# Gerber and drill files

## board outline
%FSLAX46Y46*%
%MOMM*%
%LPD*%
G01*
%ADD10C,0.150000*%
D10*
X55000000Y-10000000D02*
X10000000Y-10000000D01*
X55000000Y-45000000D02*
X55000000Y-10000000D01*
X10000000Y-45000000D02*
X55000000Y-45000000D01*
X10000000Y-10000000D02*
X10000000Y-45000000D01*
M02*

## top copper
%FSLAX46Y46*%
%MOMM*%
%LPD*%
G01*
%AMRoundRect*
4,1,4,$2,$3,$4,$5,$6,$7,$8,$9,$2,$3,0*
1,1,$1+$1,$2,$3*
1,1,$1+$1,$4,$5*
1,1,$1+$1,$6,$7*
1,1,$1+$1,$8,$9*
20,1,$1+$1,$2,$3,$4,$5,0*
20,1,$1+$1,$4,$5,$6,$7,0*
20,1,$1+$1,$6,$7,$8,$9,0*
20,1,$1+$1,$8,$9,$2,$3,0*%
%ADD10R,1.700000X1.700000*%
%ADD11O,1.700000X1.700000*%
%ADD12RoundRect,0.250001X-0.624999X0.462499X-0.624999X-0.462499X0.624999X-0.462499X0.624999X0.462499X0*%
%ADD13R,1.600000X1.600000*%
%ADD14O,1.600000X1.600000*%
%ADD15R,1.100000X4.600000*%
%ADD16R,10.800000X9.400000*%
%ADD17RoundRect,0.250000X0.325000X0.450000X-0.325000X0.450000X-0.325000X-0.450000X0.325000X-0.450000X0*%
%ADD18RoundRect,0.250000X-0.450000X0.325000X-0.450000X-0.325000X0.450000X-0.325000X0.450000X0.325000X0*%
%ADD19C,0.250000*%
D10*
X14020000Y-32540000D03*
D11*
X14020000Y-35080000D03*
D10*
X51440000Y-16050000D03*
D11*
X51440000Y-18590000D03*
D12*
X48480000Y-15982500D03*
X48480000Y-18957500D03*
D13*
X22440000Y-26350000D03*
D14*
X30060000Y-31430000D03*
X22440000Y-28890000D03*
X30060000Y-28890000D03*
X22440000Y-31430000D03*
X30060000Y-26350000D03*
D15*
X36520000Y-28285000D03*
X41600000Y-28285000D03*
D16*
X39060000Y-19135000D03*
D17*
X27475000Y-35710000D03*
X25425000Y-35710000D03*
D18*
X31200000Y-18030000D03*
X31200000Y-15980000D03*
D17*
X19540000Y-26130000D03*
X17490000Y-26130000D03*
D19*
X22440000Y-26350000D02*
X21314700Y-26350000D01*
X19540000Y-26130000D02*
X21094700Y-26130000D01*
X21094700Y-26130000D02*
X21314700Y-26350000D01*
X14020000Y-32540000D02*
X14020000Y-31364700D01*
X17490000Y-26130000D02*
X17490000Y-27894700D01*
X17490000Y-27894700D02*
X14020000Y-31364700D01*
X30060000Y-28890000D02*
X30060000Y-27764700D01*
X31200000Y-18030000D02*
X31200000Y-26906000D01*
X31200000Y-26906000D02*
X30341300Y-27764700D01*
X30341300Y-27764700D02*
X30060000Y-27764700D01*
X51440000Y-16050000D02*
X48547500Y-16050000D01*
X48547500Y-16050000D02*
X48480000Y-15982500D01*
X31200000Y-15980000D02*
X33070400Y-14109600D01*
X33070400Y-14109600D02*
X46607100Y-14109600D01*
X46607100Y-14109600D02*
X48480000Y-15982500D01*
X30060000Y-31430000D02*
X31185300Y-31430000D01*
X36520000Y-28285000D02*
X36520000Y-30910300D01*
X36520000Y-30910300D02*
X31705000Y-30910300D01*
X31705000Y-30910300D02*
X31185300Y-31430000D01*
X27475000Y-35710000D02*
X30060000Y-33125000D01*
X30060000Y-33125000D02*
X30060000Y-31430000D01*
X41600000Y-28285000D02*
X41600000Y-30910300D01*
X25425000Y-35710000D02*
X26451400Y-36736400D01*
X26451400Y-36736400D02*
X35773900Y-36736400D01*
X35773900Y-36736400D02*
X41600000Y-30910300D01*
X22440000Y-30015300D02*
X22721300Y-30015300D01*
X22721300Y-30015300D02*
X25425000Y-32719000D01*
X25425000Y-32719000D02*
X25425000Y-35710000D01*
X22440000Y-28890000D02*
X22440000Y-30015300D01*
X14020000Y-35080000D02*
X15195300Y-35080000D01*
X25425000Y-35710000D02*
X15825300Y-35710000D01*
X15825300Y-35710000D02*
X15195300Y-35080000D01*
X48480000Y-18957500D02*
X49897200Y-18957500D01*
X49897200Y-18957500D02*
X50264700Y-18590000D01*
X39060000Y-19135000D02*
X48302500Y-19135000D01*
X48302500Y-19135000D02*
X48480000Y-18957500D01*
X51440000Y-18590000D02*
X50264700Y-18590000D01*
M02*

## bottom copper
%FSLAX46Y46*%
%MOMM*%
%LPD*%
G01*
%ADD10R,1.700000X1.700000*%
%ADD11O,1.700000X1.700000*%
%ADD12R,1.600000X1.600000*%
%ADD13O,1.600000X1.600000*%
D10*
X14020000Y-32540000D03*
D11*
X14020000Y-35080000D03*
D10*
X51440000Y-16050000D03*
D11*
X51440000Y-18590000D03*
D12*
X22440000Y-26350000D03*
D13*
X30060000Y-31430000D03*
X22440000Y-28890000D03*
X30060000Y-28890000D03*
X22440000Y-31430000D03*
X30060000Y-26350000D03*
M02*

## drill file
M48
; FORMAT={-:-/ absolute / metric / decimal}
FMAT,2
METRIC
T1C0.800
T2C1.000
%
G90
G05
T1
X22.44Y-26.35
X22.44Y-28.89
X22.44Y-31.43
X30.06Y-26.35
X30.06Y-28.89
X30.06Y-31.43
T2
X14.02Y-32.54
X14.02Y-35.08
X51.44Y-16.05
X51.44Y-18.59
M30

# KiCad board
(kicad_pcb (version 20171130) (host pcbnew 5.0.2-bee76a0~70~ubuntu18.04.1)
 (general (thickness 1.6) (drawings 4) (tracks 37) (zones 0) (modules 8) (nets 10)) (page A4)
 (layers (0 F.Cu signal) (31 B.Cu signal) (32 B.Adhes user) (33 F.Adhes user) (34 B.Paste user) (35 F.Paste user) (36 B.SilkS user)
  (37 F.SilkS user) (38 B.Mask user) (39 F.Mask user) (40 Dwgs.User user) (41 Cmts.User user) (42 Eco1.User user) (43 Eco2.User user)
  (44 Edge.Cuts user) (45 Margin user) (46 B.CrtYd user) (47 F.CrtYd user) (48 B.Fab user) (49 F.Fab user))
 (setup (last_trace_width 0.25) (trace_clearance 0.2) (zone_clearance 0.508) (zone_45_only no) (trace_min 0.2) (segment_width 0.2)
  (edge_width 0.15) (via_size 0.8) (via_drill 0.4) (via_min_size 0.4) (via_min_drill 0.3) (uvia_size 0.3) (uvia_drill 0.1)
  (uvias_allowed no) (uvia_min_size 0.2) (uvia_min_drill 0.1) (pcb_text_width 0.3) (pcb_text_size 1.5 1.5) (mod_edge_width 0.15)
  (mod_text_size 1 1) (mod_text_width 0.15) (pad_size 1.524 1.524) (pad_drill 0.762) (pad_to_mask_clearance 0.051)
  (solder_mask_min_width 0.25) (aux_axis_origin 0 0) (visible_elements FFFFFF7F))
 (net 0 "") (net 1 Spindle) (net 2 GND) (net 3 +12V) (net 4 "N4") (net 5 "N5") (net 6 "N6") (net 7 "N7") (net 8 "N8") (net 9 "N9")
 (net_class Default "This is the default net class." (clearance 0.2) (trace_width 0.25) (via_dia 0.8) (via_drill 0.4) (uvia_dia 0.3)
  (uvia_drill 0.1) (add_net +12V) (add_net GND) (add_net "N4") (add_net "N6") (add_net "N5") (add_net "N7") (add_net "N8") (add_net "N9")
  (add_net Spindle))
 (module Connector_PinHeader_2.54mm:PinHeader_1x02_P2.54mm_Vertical (layer F.Cu) (at 14.02 32.54)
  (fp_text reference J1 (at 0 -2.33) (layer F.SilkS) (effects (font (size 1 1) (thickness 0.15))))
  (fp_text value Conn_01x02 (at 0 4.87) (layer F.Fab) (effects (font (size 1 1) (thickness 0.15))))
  (pad 1 thru_hole rect (at 0 0) (size 1.7 1.7) (drill 1) (layers *.Cu *.Mask) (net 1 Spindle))
  (pad 2 thru_hole oval (at 0 2.54) (size 1.7 1.7) (drill 1) (layers *.Cu *.Mask) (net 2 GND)))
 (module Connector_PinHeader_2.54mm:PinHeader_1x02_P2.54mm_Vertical (layer F.Cu) (at 51.44 16.05)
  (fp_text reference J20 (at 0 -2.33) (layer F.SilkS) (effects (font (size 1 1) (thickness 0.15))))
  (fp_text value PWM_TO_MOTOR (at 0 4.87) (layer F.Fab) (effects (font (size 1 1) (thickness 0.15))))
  (pad 1 thru_hole rect (at 0 0) (size 1.7 1.7) (drill 1) (layers *.Cu *.Mask) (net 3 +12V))
  (pad 2 thru_hole oval (at 0 2.54) (size 1.7 1.7) (drill 1) (layers *.Cu *.Mask) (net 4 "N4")))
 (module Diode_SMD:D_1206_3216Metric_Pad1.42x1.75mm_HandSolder (layer F.Cu) (at 48.48 17.47 270)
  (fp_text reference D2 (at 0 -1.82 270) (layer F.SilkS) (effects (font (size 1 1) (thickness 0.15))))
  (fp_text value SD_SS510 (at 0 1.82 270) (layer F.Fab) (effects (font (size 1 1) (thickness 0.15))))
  (pad 1 smd roundrect (at -1.4875 0 270) (size 1.425 1.75) (layers F.Cu F.Paste F.Mask) (roundrect_rratio 0.175439) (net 3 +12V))
  (pad 2 smd roundrect (at 1.4875 0 270) (size 1.425 1.75) (layers F.Cu F.Paste F.Mask) (roundrect_rratio 0.175439) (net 4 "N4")))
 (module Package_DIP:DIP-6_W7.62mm (layer F.Cu) (at 22.44 26.35)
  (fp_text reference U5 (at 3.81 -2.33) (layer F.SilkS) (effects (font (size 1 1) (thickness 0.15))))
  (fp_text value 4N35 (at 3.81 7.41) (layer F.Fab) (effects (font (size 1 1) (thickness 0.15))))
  (pad 1 thru_hole rect (at 0 0) (size 1.6 1.6) (drill 0.8) (layers *.Cu *.Mask) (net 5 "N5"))
  (pad 4 thru_hole oval (at 7.62 5.08) (size 1.6 1.6) (drill 0.8) (layers *.Cu *.Mask) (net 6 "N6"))
  (pad 2 thru_hole oval (at 0 2.54) (size 1.6 1.6) (drill 0.8) (layers *.Cu *.Mask) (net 2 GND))
  (pad 5 thru_hole oval (at 7.62 2.54) (size 1.6 1.6) (drill 0.8) (layers *.Cu *.Mask) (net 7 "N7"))
  (pad 3 thru_hole oval (at 0 5.08) (size 1.6 1.6) (drill 0.8) (layers *.Cu *.Mask) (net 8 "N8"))
  (pad 6 thru_hole oval (at 7.62 0) (size 1.6 1.6) (drill 0.8) (layers *.Cu *.Mask) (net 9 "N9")))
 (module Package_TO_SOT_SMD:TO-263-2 (layer F.Cu) (at 39.06 22.51 90)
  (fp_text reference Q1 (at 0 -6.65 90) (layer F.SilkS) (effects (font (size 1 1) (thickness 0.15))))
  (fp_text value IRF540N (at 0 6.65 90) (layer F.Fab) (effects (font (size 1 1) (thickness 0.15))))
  (pad 1 smd rect (at -5.775 -2.54 90) (size 4.6 1.1) (layers F.Cu F.Paste F.Mask) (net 6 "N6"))
  (pad 3 smd rect (at -5.775 2.54 90) (size 4.6 1.1) (layers F.Cu F.Paste F.Mask) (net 2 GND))
  (pad 2 smd rect (at 3.375 0 90) (size 9.4 10.8) (layers F.Cu F.Mask) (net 4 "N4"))
  (pad "" smd rect (at 5.8 2.775 90) (size 4.55 5.25) (layers F.Paste))
  (pad "" smd rect (at 0.95 -2.775 90) (size 4.55 5.25) (layers F.Paste))
  (pad "" smd rect (at 5.8 -2.775 90) (size 4.55 5.25) (layers F.Paste))
  (pad "" smd rect (at 0.95 2.775 90) (size 4.55 5.25) (layers F.Paste)))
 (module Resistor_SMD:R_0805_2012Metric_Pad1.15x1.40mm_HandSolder (layer F.Cu) (at 26.45 35.71 180)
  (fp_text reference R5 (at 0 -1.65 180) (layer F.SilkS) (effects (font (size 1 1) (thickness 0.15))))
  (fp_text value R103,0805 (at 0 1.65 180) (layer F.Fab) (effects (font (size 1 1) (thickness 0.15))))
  (pad 1 smd roundrect (at -1.025 0 180) (size 1.15 1.4) (layers F.Cu F.Paste F.Mask) (roundrect_rratio 0.217391) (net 6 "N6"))
  (pad 2 smd roundrect (at 1.025 0 180) (size 1.15 1.4) (layers F.Cu F.Paste F.Mask) (roundrect_rratio 0.217391) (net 2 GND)))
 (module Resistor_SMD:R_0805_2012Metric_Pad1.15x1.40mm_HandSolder (layer F.Cu) (at 31.2 17.005 270)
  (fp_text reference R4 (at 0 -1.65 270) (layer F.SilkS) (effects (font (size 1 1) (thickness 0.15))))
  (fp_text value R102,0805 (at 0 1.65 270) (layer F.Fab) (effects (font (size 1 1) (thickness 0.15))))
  (pad 2 smd roundrect (at 1.025 0 270) (size 1.15 1.4) (layers F.Cu F.Paste F.Mask) (roundrect_rratio 0.217391) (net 7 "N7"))
  (pad 1 smd roundrect (at -1.025 0 270) (size 1.15 1.4) (layers F.Cu F.Paste F.Mask) (roundrect_rratio 0.217391) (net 3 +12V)))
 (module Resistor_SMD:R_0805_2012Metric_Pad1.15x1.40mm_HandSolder (layer F.Cu) (at 18.515 26.13 180)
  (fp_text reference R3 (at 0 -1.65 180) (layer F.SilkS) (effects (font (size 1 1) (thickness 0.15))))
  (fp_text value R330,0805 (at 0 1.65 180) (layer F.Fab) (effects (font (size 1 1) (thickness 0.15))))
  (pad 1 smd roundrect (at -1.025 0 180) (size 1.15 1.4) (layers F.Cu F.Paste F.Mask) (roundrect_rratio 0.217391) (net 5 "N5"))
  (pad 2 smd roundrect (at 1.025 0 180) (size 1.15 1.4) (layers F.Cu F.Paste F.Mask) (roundrect_rratio 0.217391) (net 1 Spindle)))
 (gr_line (start 55 10) (end 10 10) (layer Edge.Cuts) (width 0.15))
 (gr_line (start 55 45) (end 55 10) (layer Edge.Cuts) (width 0.15))
 (gr_line (start 10 45) (end 55 45) (layer Edge.Cuts) (width 0.15))
 (gr_line (start 10 10) (end 10 45) (layer Edge.Cuts) (width 0.15))
 (segment (start 22.44 26.35) (end 21.3147 26.35) (width 0.25) (layer F.Cu) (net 5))
 (segment (start 19.54 26.13) (end 21.0947 26.13) (width 0.25) (layer F.Cu) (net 5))
 (segment (start 21.0947 26.13) (end 21.3147 26.35) (width 0.25) (layer F.Cu) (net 5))
 (segment (start 14.02 32.54) (end 14.02 31.3647) (width 0.25) (layer F.Cu) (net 1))
 (segment (start 17.49 26.13) (end 17.49 27.8947) (width 0.25) (layer F.Cu) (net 1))
 (segment (start 17.49 27.8947) (end 14.02 31.3647) (width 0.25) (layer F.Cu) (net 1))
 (segment (start 30.06 28.89) (end 30.06 27.7647) (width 0.25) (layer F.Cu) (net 7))
 (segment (start 31.2 18.03) (end 31.2 26.906) (width 0.25) (layer F.Cu) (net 7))
 (segment (start 31.2 26.906) (end 30.3413 27.7647) (width 0.25) (layer F.Cu) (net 7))
 (segment (start 30.3413 27.7647) (end 30.06 27.7647) (width 0.25) (layer F.Cu) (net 7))
 (segment (start 51.44 16.05) (end 48.5475 16.05) (width 0.25) (layer F.Cu) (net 3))
 (segment (start 48.5475 16.05) (end 48.48 15.9825) (width 0.25) (layer F.Cu) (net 3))
 (segment (start 31.2 15.98) (end 33.0704 14.1096) (width 0.25) (layer F.Cu) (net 3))
 (segment (start 33.0704 14.1096) (end 46.6071 14.1096) (width 0.25) (layer F.Cu) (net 3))
 (segment (start 46.6071 14.1096) (end 48.48 15.9825) (width 0.25) (layer F.Cu) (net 3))
 (segment (start 30.06 31.43) (end 31.1853 31.43) (width 0.25) (layer F.Cu) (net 6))
 (segment (start 36.52 28.285) (end 36.52 30.9103) (width 0.25) (layer F.Cu) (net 6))
 (segment (start 36.52 30.9103) (end 31.705 30.9103) (width 0.25) (layer F.Cu) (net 6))
 (segment (start 31.705 30.9103) (end 31.1853 31.43) (width 0.25) (layer F.Cu) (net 6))
 (segment (start 27.475 35.71) (end 30.06 33.125) (width 0.25) (layer F.Cu) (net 6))
 (segment (start 30.06 33.125) (end 30.06 31.43) (width 0.25) (layer F.Cu) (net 6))
 (segment (start 41.6 28.285) (end 41.6 30.9103) (width 0.25) (layer F.Cu) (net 2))
 (segment (start 25.425 35.71) (end 26.4514 36.7364) (width 0.25) (layer F.Cu) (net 2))
 (segment (start 26.4514 36.7364) (end 35.7739 36.7364) (width 0.25) (layer F.Cu) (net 2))
 (segment (start 35.7739 36.7364) (end 41.6 30.9103) (width 0.25) (layer F.Cu) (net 2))
 (segment (start 22.44 30.0153) (end 22.7213 30.0153) (width 0.25) (layer F.Cu) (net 2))
 (segment (start 22.7213 30.0153) (end 25.425 32.719) (width 0.25) (layer F.Cu) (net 2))
 (segment (start 25.425 32.719) (end 25.425 35.71) (width 0.25) (layer F.Cu) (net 2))
 (segment (start 22.44 28.89) (end 22.44 30.0153) (width 0.25) (layer F.Cu) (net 2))
 (segment (start 14.02 35.08) (end 15.1953 35.08) (width 0.25) (layer F.Cu) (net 2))
 (segment (start 25.425 35.71) (end 15.8253 35.71) (width 0.25) (layer F.Cu) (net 2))
 (segment (start 15.8253 35.71) (end 15.1953 35.08) (width 0.25) (layer F.Cu) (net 2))
 (segment (start 48.48 18.9575) (end 49.8972 18.9575) (width 0.25) (layer F.Cu) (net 4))
 (segment (start 49.8972 18.9575) (end 50.2647 18.59) (width 0.25) (layer F.Cu) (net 4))
 (segment (start 39.06 19.135) (end 48.3025 19.135) (width 0.25) (layer F.Cu) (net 4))
 (segment (start 48.3025 19.135) (end 48.48 18.9575) (width 0.25) (layer F.Cu) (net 4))
 (segment (start 51.44 18.59) (end 50.2647 18.59) (width 0.25) (layer F.Cu) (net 4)))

